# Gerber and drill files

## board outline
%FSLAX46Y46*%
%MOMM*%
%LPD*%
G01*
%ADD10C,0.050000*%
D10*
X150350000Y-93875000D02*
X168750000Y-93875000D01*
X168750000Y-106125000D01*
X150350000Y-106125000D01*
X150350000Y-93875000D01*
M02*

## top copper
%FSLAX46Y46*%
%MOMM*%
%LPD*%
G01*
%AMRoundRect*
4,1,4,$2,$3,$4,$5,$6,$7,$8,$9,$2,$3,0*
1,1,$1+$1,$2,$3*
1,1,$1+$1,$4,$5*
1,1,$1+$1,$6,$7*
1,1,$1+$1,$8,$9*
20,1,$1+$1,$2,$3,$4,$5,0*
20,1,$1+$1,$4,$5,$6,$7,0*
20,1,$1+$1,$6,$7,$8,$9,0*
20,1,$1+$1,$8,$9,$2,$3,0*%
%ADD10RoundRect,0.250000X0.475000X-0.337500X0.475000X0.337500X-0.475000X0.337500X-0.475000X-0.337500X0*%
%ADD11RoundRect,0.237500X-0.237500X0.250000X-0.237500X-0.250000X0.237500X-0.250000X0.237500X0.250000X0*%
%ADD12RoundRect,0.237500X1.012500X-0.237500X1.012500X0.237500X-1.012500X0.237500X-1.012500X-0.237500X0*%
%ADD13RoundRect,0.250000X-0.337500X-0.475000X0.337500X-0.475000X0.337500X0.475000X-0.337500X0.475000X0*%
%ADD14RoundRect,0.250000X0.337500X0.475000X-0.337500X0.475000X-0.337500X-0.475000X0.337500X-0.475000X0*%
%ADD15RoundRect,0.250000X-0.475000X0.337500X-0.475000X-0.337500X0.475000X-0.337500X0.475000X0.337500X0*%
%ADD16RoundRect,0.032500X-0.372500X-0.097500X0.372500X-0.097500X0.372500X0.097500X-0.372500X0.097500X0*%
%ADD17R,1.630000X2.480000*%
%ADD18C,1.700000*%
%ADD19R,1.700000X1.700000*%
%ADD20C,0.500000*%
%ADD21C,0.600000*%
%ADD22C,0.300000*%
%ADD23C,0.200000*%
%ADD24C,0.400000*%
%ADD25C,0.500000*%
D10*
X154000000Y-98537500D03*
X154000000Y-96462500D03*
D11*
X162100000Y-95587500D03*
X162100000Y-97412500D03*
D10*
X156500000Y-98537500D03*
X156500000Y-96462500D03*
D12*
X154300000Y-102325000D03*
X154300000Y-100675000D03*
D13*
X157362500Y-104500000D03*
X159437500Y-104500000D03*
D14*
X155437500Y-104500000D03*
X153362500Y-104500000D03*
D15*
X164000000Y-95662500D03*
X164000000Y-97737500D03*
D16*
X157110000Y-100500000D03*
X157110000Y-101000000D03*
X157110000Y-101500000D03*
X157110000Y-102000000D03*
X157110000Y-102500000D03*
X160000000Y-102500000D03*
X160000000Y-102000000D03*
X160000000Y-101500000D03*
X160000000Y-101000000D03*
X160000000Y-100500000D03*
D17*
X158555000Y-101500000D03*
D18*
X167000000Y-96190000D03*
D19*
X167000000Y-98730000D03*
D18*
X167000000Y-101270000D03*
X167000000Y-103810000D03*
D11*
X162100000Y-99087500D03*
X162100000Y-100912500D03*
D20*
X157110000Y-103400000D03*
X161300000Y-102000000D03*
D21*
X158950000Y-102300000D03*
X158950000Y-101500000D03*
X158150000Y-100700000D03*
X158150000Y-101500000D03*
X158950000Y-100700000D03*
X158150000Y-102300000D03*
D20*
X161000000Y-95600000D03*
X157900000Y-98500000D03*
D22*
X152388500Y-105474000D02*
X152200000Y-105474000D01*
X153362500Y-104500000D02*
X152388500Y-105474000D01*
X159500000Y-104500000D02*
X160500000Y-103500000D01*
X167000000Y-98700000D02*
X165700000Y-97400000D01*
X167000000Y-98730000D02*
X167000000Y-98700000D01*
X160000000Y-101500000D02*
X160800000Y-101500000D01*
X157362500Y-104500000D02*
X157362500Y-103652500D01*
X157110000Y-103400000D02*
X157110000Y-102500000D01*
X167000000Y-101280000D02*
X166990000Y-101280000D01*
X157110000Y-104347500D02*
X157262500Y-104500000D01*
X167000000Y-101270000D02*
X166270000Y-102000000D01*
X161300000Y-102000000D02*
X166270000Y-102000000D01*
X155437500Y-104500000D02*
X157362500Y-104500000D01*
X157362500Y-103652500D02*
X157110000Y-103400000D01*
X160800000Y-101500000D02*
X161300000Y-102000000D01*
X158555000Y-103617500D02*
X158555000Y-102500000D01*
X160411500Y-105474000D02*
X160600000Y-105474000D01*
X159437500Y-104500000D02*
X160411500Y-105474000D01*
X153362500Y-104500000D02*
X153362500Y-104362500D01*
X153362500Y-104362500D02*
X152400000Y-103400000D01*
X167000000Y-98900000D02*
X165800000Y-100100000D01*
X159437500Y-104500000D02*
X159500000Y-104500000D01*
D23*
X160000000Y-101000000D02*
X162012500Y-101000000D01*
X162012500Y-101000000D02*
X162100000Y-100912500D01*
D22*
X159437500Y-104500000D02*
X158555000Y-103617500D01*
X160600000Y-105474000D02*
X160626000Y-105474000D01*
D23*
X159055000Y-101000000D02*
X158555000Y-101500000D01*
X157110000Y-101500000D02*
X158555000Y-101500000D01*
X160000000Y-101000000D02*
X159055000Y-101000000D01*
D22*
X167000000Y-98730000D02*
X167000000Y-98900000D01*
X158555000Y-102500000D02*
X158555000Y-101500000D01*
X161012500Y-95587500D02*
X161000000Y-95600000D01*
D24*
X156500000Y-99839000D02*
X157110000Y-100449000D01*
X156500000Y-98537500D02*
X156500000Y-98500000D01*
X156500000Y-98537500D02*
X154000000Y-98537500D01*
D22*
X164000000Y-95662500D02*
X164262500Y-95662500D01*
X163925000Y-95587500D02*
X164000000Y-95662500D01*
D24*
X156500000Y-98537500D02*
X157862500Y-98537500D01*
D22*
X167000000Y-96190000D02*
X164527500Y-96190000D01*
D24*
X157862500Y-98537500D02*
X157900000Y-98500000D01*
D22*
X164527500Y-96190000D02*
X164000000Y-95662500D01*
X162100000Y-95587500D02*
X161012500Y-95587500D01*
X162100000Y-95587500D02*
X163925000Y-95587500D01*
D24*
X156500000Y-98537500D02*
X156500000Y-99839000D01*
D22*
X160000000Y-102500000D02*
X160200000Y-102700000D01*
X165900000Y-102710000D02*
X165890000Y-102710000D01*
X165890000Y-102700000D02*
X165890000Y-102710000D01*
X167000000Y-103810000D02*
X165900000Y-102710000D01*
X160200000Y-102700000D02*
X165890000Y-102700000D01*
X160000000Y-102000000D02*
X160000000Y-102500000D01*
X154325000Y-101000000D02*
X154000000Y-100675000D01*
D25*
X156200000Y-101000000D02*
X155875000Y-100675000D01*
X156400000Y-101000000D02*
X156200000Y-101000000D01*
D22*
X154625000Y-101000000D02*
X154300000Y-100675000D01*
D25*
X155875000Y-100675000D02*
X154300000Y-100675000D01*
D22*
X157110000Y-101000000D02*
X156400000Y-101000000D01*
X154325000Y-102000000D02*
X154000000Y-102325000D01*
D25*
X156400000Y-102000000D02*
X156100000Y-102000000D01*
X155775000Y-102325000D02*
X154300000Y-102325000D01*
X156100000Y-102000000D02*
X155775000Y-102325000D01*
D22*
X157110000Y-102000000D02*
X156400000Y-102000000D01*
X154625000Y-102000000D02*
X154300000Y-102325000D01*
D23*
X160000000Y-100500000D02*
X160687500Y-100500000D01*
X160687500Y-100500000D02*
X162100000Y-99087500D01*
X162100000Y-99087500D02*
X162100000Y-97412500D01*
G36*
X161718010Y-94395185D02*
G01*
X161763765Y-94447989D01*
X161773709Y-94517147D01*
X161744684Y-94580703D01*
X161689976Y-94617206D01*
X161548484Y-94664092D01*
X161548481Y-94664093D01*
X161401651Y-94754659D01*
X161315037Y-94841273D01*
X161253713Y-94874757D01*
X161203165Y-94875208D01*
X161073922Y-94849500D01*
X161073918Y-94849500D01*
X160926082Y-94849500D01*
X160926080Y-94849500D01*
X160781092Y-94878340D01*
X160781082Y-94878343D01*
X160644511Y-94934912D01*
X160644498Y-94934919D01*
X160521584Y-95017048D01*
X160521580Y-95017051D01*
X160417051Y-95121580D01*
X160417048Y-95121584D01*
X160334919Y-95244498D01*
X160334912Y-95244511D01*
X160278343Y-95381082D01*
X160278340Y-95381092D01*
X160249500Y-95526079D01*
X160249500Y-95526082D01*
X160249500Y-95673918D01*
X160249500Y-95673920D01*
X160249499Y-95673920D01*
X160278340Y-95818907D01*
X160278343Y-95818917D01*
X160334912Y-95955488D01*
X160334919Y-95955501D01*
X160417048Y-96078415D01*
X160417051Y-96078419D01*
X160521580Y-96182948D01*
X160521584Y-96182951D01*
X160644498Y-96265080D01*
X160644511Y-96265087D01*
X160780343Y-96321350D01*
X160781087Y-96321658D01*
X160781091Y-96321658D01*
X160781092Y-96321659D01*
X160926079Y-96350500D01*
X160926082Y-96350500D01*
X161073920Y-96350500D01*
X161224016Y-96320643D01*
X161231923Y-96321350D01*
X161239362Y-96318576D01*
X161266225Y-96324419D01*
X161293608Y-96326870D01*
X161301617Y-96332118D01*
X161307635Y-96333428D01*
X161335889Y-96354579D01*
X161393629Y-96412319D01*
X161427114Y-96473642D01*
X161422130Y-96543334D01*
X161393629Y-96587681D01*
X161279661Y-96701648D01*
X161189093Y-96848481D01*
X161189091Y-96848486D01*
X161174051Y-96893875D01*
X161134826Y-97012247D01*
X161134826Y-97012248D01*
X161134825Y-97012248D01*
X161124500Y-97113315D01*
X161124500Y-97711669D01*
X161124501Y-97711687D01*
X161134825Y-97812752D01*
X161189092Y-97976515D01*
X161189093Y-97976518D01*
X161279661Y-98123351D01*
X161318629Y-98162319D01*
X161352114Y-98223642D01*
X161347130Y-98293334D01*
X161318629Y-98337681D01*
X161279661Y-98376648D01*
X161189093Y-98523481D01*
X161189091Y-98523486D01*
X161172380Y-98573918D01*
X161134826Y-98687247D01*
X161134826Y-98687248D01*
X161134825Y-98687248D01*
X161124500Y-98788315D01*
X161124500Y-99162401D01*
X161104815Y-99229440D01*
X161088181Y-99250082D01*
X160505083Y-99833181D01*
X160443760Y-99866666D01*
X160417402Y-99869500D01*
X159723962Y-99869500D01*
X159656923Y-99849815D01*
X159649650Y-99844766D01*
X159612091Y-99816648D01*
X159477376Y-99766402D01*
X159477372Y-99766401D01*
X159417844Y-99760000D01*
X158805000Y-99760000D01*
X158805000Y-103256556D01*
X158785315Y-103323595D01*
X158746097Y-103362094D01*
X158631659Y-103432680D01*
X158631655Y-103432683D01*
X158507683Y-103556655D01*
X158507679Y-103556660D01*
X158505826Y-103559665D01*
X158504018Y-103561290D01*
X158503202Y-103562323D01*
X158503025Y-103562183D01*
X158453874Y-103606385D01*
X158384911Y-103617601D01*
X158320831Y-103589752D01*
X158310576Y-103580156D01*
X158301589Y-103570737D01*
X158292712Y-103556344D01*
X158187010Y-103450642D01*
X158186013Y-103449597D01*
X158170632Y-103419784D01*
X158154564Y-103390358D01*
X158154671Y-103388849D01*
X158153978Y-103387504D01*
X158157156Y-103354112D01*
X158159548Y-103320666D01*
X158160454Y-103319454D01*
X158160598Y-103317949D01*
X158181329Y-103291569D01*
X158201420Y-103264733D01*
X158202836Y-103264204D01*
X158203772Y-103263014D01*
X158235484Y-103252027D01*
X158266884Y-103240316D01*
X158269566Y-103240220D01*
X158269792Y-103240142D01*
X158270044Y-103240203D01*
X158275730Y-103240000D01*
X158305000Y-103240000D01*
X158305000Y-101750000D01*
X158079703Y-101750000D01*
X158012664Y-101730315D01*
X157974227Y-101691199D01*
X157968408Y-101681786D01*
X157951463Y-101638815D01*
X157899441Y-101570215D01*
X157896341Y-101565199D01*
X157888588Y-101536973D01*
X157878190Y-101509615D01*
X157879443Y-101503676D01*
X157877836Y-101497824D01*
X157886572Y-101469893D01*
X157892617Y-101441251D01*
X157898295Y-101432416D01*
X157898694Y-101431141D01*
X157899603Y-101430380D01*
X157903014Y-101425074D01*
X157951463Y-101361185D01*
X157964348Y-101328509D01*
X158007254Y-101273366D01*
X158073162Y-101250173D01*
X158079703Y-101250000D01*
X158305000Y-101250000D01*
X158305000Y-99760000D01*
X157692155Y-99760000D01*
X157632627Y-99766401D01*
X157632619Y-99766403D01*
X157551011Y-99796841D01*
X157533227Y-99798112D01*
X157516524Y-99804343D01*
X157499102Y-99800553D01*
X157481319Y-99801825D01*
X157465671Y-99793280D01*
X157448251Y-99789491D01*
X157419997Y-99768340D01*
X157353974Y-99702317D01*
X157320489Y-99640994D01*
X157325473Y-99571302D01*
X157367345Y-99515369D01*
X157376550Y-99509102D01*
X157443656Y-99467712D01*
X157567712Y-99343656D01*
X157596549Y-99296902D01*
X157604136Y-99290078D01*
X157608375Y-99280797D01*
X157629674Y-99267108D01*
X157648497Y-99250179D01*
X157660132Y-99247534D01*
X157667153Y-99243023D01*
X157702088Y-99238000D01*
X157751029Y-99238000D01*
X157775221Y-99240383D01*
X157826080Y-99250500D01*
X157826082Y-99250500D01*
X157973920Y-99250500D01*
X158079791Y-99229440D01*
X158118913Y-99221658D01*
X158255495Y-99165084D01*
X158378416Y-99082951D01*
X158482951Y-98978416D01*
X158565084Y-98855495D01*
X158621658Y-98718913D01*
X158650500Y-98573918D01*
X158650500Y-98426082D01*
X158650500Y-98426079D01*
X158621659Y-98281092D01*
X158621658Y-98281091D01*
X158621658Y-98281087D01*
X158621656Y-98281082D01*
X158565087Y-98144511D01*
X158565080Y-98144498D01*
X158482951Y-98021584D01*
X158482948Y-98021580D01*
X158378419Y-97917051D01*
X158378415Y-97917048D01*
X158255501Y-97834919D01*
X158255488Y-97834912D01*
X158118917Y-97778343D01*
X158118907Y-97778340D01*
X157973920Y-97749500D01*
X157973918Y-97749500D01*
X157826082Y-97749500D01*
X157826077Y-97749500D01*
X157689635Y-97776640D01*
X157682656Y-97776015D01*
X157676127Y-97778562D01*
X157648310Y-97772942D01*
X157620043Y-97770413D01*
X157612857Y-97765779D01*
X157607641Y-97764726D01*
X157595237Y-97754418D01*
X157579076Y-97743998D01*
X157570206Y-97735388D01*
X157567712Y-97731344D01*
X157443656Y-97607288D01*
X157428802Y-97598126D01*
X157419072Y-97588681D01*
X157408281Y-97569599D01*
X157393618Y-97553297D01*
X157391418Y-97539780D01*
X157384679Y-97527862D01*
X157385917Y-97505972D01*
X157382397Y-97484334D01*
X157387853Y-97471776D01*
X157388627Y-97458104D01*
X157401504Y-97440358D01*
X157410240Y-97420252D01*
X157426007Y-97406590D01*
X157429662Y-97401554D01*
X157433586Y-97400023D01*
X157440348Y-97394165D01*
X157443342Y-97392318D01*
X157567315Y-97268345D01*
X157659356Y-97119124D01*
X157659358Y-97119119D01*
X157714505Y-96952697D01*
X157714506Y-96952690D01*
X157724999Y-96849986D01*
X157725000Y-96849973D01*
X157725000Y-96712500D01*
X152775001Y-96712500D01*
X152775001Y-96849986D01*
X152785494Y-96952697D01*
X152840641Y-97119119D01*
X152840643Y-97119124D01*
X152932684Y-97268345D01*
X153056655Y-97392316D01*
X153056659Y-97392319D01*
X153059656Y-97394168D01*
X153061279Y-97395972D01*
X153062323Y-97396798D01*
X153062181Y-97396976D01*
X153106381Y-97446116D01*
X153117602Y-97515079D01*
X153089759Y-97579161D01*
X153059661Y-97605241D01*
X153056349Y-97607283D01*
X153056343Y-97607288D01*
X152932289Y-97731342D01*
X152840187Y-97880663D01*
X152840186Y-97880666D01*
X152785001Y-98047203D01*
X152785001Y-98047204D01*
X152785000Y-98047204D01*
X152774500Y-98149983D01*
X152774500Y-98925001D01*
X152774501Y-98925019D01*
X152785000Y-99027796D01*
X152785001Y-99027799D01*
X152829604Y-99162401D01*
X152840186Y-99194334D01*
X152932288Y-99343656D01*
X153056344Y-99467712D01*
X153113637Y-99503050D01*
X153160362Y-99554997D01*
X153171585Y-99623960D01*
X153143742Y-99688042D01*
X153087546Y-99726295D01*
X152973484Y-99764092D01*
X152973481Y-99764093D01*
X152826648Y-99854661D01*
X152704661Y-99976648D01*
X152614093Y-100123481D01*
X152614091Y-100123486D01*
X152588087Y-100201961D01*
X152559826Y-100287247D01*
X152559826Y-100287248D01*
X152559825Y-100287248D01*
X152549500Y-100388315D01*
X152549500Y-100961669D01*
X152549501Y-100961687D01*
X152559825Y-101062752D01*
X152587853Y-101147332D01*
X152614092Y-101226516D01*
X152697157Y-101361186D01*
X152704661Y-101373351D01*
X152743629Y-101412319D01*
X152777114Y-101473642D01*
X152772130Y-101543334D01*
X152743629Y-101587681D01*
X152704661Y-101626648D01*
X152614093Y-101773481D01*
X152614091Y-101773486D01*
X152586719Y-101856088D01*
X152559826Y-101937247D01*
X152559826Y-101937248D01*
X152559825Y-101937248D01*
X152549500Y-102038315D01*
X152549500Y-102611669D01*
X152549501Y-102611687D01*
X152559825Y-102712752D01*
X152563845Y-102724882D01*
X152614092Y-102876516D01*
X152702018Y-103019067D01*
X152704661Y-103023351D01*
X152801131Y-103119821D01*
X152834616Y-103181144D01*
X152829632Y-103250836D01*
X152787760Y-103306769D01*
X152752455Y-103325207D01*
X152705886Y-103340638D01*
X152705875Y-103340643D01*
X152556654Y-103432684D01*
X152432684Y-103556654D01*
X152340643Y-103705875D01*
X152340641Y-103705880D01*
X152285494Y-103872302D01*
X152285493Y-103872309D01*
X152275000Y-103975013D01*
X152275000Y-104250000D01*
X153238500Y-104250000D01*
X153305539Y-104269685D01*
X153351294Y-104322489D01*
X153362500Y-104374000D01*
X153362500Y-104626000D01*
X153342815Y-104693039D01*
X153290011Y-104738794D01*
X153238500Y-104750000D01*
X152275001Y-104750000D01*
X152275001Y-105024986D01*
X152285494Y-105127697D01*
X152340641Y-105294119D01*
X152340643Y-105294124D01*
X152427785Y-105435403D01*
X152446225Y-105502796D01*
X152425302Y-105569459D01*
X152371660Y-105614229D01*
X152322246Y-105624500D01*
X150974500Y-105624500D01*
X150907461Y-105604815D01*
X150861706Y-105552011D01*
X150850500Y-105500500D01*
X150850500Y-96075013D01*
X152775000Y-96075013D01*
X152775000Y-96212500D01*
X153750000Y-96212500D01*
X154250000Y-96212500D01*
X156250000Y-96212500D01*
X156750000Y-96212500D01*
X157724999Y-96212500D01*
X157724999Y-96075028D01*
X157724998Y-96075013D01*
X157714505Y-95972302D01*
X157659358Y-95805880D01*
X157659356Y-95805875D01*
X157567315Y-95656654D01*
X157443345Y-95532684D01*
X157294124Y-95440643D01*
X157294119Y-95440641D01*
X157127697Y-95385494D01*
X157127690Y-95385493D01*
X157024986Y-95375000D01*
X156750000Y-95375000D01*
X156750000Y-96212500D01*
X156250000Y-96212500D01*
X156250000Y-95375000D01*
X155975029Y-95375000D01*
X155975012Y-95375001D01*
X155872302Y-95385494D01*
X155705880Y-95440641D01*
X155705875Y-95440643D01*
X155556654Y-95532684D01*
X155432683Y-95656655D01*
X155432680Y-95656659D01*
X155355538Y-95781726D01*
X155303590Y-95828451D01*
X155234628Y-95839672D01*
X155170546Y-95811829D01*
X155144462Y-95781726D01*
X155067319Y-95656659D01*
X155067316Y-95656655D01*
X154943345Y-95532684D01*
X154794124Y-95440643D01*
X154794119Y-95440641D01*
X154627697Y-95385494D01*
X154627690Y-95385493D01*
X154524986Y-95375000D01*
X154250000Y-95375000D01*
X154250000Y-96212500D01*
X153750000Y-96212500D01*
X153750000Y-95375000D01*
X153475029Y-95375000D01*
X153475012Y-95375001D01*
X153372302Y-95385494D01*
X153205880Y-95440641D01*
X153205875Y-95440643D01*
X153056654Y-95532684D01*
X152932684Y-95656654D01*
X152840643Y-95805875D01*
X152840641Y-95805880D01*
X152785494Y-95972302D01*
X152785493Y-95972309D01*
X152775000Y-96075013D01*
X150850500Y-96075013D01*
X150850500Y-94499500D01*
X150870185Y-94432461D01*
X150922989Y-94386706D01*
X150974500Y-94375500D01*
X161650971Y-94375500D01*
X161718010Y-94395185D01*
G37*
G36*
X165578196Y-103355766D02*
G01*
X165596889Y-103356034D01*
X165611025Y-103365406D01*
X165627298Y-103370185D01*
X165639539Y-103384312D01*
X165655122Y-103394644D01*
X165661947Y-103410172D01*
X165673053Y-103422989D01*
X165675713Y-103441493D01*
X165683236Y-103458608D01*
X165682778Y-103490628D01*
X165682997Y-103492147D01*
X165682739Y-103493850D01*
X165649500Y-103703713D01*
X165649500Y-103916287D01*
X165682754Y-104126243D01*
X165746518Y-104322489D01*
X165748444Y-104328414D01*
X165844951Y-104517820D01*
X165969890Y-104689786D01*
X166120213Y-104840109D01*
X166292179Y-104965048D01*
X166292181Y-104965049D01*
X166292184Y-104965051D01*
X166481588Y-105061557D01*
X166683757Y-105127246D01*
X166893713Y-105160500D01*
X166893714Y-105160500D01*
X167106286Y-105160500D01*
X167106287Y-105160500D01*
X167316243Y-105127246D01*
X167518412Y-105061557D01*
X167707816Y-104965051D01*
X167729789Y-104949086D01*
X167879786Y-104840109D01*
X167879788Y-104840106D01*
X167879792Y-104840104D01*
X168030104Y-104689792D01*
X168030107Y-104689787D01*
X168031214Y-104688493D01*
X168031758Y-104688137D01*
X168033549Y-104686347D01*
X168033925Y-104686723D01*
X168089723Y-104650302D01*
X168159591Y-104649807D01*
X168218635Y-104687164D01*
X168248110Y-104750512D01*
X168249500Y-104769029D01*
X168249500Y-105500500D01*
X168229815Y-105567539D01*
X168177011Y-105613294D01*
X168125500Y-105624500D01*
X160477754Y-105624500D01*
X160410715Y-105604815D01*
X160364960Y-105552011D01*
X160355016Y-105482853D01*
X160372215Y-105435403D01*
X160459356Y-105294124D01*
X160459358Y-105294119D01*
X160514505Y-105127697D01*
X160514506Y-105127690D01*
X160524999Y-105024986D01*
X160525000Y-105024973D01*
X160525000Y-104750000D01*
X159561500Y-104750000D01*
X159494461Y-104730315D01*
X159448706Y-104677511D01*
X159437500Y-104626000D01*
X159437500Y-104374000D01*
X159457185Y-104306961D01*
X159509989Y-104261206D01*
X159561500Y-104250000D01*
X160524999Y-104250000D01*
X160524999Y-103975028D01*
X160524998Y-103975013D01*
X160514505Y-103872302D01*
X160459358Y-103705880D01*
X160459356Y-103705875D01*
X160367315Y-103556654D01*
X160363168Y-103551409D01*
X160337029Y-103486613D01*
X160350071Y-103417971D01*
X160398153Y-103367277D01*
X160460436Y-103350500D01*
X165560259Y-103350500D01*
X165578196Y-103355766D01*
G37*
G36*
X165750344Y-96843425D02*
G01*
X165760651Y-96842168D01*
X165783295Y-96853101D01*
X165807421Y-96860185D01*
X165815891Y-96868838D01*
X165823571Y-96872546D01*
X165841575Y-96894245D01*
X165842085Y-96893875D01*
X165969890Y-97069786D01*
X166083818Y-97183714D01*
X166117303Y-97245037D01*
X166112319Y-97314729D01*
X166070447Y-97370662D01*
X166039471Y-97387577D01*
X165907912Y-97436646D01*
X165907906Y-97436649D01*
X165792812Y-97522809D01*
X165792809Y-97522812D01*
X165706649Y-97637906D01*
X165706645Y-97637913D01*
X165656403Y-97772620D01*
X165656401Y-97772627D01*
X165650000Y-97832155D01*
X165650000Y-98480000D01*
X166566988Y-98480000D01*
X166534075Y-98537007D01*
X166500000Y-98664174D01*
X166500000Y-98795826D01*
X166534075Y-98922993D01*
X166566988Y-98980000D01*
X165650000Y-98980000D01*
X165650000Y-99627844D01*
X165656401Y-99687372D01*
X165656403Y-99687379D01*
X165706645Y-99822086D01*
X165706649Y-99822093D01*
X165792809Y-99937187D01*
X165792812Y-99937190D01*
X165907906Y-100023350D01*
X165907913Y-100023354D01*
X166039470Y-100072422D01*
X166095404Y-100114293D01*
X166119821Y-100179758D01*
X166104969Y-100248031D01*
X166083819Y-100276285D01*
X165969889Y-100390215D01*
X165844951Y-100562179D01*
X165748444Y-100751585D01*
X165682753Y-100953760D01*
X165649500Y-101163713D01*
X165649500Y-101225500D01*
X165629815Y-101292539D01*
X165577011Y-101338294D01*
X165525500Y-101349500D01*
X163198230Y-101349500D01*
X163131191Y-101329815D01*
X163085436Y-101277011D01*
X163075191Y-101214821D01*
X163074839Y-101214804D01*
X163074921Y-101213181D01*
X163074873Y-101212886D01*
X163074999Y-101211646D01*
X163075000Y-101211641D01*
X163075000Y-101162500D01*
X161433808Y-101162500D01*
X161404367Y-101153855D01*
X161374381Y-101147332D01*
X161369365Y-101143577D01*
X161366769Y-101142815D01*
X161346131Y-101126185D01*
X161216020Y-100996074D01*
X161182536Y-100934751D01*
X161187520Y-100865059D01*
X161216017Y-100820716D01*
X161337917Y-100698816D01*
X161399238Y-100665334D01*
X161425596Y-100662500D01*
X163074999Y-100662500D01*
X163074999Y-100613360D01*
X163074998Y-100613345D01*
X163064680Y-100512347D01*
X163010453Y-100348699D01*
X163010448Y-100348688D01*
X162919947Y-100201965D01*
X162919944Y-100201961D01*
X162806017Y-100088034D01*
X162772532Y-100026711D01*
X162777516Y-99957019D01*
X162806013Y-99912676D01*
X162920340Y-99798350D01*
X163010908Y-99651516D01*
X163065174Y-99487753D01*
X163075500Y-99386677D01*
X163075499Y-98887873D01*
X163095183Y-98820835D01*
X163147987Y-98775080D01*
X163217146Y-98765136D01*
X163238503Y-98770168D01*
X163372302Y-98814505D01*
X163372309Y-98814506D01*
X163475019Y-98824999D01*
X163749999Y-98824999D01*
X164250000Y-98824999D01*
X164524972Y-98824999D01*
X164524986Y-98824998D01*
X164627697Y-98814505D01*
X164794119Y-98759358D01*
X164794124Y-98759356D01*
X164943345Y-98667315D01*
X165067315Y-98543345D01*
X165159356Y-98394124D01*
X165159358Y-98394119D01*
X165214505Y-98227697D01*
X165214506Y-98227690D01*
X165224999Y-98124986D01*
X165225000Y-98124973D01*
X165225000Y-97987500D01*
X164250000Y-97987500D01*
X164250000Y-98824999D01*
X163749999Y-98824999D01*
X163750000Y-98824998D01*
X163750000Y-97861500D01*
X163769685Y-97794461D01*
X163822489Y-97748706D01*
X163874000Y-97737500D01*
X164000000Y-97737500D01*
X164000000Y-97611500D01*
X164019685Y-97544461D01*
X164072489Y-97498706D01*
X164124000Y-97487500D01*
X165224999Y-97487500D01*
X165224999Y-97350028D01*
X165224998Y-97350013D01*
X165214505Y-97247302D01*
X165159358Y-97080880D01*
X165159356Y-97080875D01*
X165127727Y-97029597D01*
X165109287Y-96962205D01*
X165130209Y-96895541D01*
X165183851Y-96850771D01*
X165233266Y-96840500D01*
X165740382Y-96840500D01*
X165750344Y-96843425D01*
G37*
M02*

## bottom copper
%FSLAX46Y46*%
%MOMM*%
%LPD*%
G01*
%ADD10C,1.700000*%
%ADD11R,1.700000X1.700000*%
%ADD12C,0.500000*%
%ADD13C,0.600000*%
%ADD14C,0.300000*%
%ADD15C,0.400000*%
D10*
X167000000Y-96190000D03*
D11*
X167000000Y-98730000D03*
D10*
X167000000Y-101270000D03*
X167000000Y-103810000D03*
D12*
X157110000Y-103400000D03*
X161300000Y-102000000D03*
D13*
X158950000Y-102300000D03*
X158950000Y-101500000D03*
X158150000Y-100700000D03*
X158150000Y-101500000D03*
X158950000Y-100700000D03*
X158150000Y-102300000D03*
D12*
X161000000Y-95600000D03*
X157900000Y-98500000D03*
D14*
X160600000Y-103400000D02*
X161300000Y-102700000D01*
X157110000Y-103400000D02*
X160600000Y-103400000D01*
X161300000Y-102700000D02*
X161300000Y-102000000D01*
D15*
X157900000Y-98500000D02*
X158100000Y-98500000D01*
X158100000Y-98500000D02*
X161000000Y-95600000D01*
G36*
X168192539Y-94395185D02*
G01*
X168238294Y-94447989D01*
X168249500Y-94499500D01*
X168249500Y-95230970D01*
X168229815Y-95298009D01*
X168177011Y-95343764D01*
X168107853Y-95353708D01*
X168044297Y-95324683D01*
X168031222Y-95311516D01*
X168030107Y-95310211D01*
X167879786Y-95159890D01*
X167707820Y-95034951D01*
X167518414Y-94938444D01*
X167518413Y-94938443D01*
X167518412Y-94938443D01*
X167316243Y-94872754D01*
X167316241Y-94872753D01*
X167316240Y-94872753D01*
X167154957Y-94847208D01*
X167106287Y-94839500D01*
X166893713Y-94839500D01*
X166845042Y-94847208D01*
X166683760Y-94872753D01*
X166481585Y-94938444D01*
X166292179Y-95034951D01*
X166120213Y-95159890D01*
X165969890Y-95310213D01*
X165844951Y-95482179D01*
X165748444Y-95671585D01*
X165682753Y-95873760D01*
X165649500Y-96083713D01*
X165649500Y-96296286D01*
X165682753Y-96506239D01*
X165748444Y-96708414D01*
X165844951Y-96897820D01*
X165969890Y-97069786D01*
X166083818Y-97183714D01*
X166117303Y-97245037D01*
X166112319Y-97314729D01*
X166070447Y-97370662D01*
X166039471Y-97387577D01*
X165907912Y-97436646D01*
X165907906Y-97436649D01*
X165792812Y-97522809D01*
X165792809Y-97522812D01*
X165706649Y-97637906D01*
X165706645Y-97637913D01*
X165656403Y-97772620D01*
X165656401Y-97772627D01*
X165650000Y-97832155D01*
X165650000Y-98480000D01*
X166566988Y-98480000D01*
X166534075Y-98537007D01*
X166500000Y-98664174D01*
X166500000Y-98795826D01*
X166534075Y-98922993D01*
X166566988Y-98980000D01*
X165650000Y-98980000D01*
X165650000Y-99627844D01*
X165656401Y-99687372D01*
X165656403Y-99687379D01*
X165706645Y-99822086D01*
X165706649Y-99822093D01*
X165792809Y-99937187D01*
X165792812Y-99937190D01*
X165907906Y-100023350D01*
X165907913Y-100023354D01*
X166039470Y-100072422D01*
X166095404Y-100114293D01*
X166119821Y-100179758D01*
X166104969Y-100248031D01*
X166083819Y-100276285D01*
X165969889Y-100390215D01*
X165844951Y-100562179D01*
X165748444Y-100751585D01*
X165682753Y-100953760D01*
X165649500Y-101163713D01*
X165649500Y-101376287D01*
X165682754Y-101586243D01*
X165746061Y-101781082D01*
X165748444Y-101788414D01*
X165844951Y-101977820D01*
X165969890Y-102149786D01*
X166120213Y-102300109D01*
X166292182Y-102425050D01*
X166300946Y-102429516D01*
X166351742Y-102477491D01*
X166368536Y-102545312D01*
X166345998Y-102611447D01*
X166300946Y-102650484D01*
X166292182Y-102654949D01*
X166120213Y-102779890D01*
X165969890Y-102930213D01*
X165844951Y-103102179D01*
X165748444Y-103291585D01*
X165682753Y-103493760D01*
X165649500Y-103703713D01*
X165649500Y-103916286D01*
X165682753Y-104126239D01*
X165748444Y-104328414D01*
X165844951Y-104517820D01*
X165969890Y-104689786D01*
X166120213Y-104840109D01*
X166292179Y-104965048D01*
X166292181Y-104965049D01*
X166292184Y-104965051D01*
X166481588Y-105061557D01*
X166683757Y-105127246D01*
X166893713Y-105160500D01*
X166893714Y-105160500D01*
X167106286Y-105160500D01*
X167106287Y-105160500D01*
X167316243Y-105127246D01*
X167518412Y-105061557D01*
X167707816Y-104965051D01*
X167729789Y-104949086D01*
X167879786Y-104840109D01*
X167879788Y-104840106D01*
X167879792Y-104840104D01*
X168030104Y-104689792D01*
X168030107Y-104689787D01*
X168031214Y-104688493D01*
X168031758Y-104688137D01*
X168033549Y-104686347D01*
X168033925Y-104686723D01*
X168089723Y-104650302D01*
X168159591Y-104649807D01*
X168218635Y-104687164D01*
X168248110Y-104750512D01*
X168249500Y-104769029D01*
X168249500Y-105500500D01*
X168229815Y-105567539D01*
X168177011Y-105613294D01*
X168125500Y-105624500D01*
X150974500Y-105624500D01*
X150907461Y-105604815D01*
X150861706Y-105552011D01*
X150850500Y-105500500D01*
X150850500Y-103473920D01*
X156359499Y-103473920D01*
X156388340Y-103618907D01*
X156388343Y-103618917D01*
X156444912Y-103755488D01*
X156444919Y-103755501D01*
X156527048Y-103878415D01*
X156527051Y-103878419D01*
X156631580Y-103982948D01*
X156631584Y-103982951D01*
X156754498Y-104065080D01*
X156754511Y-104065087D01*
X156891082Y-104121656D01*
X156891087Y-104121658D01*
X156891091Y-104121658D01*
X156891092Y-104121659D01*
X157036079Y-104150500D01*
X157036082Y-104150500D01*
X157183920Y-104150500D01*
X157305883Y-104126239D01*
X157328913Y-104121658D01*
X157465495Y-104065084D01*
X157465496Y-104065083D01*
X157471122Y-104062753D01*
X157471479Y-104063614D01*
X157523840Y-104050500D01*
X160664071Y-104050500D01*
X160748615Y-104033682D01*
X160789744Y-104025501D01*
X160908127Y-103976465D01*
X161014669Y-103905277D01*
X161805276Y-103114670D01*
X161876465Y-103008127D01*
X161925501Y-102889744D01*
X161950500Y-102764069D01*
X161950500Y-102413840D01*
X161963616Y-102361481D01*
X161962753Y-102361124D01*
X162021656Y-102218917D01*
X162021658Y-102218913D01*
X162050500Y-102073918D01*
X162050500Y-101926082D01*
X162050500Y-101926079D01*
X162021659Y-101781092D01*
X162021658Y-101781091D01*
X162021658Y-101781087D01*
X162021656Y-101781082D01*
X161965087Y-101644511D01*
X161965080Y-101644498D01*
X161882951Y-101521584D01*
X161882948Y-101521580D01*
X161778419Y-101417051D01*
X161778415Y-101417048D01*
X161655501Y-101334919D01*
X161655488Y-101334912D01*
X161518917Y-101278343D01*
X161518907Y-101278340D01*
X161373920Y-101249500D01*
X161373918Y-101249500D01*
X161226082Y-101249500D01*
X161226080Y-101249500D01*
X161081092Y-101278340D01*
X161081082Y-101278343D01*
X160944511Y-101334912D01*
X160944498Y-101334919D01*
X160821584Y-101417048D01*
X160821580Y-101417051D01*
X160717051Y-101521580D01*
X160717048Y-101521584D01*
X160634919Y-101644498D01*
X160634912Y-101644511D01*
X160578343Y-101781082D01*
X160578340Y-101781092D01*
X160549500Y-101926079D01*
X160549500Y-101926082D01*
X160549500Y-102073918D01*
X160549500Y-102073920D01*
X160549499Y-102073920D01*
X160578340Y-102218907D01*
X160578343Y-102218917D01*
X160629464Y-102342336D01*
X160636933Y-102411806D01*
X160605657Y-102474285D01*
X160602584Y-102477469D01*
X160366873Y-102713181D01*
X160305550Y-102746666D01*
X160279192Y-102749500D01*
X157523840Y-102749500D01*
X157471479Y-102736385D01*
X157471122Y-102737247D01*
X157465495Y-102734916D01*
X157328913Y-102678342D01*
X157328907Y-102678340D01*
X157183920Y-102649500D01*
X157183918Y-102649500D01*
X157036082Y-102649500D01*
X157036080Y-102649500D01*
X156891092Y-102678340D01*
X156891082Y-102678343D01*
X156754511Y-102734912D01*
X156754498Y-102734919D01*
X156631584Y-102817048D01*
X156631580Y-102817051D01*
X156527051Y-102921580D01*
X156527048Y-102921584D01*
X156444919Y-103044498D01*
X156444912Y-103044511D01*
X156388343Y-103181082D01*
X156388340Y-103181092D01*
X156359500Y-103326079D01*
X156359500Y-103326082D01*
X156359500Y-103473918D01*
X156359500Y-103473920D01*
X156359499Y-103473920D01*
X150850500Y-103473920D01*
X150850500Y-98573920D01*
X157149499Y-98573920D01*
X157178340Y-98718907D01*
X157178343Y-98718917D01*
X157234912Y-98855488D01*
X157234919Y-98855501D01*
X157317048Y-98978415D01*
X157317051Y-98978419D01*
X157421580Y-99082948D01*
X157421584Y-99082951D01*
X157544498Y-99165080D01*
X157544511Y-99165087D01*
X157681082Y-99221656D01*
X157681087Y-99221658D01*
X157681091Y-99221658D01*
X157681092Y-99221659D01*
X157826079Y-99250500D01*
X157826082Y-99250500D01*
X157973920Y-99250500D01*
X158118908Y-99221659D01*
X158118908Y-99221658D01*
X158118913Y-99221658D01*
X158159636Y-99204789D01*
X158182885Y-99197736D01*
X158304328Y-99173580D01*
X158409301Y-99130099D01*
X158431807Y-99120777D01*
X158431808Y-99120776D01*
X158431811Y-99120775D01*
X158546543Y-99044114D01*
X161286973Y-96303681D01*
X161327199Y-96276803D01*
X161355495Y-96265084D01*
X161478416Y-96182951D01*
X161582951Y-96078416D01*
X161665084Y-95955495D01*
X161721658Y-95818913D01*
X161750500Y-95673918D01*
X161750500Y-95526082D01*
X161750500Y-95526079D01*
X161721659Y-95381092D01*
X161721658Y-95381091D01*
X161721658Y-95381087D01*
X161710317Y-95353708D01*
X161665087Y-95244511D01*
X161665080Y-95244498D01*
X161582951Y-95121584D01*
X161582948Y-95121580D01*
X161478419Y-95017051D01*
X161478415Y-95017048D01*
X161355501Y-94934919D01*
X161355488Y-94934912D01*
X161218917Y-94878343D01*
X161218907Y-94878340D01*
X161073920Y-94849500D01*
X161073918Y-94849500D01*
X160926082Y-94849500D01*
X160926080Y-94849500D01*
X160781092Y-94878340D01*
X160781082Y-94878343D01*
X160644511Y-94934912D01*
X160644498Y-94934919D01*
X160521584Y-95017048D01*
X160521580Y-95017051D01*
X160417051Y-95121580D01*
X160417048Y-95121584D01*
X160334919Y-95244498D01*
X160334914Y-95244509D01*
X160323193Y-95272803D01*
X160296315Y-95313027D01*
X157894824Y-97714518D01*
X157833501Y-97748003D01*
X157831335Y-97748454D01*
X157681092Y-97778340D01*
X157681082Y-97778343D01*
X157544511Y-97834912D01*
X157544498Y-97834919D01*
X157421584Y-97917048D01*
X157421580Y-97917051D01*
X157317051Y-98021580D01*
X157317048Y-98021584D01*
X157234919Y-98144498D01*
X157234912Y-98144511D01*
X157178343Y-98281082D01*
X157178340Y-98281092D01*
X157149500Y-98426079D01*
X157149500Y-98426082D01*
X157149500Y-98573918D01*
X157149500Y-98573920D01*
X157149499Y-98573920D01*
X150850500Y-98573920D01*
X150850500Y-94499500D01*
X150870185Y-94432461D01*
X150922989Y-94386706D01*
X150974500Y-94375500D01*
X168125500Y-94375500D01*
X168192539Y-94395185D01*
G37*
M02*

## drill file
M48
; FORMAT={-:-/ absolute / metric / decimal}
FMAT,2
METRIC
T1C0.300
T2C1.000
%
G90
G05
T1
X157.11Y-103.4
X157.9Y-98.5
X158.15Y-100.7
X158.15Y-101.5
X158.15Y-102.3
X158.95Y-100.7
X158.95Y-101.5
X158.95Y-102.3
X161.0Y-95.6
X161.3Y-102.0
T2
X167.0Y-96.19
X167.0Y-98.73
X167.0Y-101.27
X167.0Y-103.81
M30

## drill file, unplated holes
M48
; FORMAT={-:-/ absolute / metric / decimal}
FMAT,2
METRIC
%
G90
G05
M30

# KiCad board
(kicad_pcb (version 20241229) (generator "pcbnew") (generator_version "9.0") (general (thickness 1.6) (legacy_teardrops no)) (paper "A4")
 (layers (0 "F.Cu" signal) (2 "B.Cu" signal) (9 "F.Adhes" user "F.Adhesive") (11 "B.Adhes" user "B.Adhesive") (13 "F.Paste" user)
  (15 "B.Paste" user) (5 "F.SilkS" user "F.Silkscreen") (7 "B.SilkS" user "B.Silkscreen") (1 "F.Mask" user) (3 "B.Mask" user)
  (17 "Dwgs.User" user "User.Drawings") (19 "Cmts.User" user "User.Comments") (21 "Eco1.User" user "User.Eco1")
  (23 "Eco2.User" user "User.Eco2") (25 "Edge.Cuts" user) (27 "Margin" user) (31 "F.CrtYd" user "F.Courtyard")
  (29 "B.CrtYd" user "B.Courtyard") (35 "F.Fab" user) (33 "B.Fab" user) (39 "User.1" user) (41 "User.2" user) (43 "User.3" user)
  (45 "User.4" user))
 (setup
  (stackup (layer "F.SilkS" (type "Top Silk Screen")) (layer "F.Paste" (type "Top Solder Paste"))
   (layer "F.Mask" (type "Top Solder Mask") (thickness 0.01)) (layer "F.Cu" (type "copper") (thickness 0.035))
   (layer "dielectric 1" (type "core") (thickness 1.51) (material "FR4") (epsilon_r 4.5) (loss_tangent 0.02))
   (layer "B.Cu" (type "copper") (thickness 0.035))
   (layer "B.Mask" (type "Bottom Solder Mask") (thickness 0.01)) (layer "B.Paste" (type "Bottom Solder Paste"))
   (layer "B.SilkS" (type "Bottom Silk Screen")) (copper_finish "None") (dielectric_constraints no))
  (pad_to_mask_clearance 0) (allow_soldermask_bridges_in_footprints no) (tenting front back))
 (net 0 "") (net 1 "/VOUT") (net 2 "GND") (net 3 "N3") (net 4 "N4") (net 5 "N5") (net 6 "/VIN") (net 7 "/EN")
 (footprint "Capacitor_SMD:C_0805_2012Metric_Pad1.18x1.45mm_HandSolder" (layer "F.Cu") (at 154 97.5 90)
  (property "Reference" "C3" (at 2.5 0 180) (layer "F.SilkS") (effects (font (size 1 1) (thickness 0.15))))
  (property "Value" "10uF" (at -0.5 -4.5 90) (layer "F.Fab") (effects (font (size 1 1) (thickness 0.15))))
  (pad "1" smd roundrect (at -1.0375 0 90) (size 1.175 1.45) (layers "F.Cu" "F.Mask" "F.Paste") (roundrect_rratio 0.212766) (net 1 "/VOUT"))
  (pad "2" smd roundrect (at 1.0375 0 90) (size 1.175 1.45) (layers "F.Cu" "F.Mask" "F.Paste") (roundrect_rratio 0.212766) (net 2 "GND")))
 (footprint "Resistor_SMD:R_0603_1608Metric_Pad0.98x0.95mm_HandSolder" (layer "F.Cu") (at 162.1 96.5 -90)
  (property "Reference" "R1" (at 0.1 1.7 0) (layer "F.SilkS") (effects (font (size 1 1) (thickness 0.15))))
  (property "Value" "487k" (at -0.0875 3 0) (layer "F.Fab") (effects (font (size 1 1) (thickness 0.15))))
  (pad "1" smd roundrect (at -0.9125 0 270) (size 0.975 0.95) (layers "F.Cu" "F.Mask" "F.Paste") (roundrect_rratio 0.25) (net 1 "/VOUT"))
  (pad "2" smd roundrect (at 0.9125 0 270) (size 0.975 0.95) (layers "F.Cu" "F.Mask" "F.Paste") (roundrect_rratio 0.25) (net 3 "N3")))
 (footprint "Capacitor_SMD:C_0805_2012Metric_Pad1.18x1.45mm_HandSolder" (layer "F.Cu") (at 156.5 97.5 90)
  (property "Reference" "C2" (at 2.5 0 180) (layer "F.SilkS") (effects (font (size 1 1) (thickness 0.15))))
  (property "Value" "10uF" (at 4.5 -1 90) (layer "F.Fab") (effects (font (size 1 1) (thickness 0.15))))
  (pad "1" smd roundrect (at -1.0375 0 90) (size 1.175 1.45) (layers "F.Cu" "F.Mask" "F.Paste") (roundrect_rratio 0.212766) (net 1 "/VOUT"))
  (pad "2" smd roundrect (at 1.0375 0 90) (size 1.175 1.45) (layers "F.Cu" "F.Mask" "F.Paste") (roundrect_rratio 0.212766) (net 2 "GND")))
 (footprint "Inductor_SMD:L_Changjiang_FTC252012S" (layer "F.Cu") (at 154.3 101.5 90)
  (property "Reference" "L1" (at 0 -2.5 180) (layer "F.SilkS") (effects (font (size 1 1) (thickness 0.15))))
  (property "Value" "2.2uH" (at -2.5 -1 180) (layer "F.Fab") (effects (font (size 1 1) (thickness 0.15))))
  (pad "1" smd roundrect (at -0.825 0 90) (size 0.95 2.5) (layers "F.Cu" "F.Mask" "F.Paste") (roundrect_rratio 0.25) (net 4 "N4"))
  (pad "2" smd roundrect (at 0.825 0 90) (size 0.95 2.5) (layers "F.Cu" "F.Mask" "F.Paste") (roundrect_rratio 0.25) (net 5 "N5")))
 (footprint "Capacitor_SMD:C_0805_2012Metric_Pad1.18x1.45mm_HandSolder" (layer "F.Cu") (at 158.4 104.5)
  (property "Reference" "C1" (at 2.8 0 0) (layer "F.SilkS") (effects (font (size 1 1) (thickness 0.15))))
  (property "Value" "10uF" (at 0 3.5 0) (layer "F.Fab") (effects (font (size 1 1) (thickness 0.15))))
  (pad "1" smd roundrect (at -1.0375 0) (size 1.175 1.45) (layers "F.Cu" "F.Mask" "F.Paste") (roundrect_rratio 0.212766) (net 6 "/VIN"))
  (pad "2" smd roundrect (at 1.0375 0) (size 1.175 1.45) (layers "F.Cu" "F.Mask" "F.Paste") (roundrect_rratio 0.212766) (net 2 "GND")))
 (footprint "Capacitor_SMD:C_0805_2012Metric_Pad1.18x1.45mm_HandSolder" (layer "F.Cu") (at 154.4 104.5 180)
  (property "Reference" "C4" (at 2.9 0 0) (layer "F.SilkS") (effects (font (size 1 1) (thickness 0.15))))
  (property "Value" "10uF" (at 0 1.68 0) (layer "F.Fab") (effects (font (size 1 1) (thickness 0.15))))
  (pad "1" smd roundrect (at -1.0375 0 180) (size 1.175 1.45) (layers "F.Cu" "F.Mask" "F.Paste") (roundrect_rratio 0.212766) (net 6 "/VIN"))
  (pad "2" smd roundrect (at 1.0375 0 180) (size 1.175 1.45) (layers "F.Cu" "F.Mask" "F.Paste") (roundrect_rratio 0.212766) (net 2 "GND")))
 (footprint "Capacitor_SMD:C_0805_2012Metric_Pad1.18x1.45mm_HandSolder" (layer "F.Cu") (at 164 96.7 -90)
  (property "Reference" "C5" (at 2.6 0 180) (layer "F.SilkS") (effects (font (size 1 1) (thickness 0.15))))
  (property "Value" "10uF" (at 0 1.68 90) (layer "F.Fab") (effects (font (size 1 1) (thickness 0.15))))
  (pad "1" smd roundrect (at -1.0375 0 270) (size 1.175 1.45) (layers "F.Cu" "F.Mask" "F.Paste") (roundrect_rratio 0.212766) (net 1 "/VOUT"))
  (pad "2" smd roundrect (at 1.0375 0 270) (size 1.175 1.45) (layers "F.Cu" "F.Mask" "F.Paste") (roundrect_rratio 0.212766) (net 2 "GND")))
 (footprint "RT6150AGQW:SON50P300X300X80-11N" (layer "F.Cu") (at 158.555 101.5)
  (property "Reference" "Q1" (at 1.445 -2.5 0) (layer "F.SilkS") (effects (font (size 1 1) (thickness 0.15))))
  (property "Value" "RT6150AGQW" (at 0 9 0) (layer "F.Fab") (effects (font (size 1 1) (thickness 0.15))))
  (pad "1" smd roundrect (at -1.445 -1) (size 0.81 0.26) (layers "F.Cu" "F.Mask" "F.Paste") (roundrect_rratio 0.125) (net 1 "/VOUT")
   (solder_mask_margin 0.102))
  (pad "2" smd roundrect (at -1.445 -0.5) (size 0.81 0.26) (layers "F.Cu" "F.Mask" "F.Paste") (roundrect_rratio 0.125) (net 5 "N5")
   (solder_mask_margin 0.102))
  (pad "3" smd roundrect (at -1.445 0) (size 0.81 0.26) (layers "F.Cu" "F.Mask" "F.Paste") (roundrect_rratio 0.125) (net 2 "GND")
   (solder_mask_margin 0.102))
  (pad "4" smd roundrect (at -1.445 0.5) (size 0.81 0.26) (layers "F.Cu" "F.Mask" "F.Paste") (roundrect_rratio 0.125) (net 4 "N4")
   (solder_mask_margin 0.102))
  (pad "5" smd roundrect (at -1.445 1) (size 0.81 0.26) (layers "F.Cu" "F.Mask" "F.Paste") (roundrect_rratio 0.125) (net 6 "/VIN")
   (solder_mask_margin 0.102))
  (pad "6" smd roundrect (at 1.445 1) (size 0.81 0.26) (layers "F.Cu" "F.Mask" "F.Paste") (roundrect_rratio 0.125) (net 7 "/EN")
   (solder_mask_margin 0.102))
  (pad "7" smd roundrect (at 1.445 0.5) (size 0.81 0.26) (layers "F.Cu" "F.Mask" "F.Paste") (roundrect_rratio 0.125) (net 7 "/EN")
   (solder_mask_margin 0.102))
  (pad "8" smd roundrect (at 1.445 0) (size 0.81 0.26) (layers "F.Cu" "F.Mask" "F.Paste") (roundrect_rratio 0.125) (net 6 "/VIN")
   (solder_mask_margin 0.102))
  (pad "9" smd roundrect (at 1.445 -0.5) (size 0.81 0.26) (layers "F.Cu" "F.Mask" "F.Paste") (roundrect_rratio 0.125) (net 2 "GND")
   (solder_mask_margin 0.102))
  (pad "10" smd roundrect (at 1.445 -1) (size 0.81 0.26) (layers "F.Cu" "F.Mask" "F.Paste") (roundrect_rratio 0.125) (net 3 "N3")
   (solder_mask_margin 0.102))
  (pad "11" smd rect (at 0 0) (size 1.63 2.48) (layers "F.Cu" "F.Mask") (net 2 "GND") (solder_mask_margin 0.102)))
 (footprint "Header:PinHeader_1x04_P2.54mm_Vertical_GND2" (layer "F.Cu") (at 167 96.19)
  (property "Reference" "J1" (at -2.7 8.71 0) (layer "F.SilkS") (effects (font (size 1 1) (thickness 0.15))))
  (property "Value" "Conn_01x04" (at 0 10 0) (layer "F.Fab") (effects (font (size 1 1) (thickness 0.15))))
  (pad "1" thru_hole circle (at 0 0) (size 1.7 1.7) (drill 1) (layers "*.Cu" "*.Mask") (remove_unused_layers no) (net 1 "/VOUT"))
  (pad "2" thru_hole rect (at 0 2.54) (size 1.7 1.7) (drill 1) (layers "*.Cu" "*.Mask") (remove_unused_layers no) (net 2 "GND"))
  (pad "3" thru_hole circle (at 0 5.08) (size 1.7 1.7) (drill 1) (layers "*.Cu" "*.Mask") (remove_unused_layers no) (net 6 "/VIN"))
  (pad "4" thru_hole circle (at 0 7.62) (size 1.7 1.7) (drill 1) (layers "*.Cu" "*.Mask") (remove_unused_layers no) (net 7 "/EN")))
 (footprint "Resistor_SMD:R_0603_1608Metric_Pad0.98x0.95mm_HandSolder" (layer "F.Cu") (at 162.1 100 -90)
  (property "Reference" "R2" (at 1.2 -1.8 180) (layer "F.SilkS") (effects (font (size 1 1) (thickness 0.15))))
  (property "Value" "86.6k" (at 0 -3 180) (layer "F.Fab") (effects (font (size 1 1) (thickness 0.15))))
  (pad "1" smd roundrect (at -0.9125 0 270) (size 0.975 0.95) (layers "F.Cu" "F.Mask" "F.Paste") (roundrect_rratio 0.25) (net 3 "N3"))
  (pad "2" smd roundrect (at 0.9125 0 270) (size 0.975 0.95) (layers "F.Cu" "F.Mask" "F.Paste") (roundrect_rratio 0.25) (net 2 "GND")))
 (gr_rect (start 150.35 93.875) (end 168.75 106.125) (stroke (width 0.05) (type default)) (fill no) (layer "Edge.Cuts"))
 (segment (start 160 101.5) (end 160.8 101.5) (width 0.3) (layer "F.Cu") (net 6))
 (segment (start 157.3625 104.5) (end 157.3625 103.6525) (width 0.3) (layer "F.Cu") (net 6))
 (segment (start 157.11 103.4) (end 157.11 102.5) (width 0.3) (layer "F.Cu") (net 6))
 (segment (start 167 101.28) (end 166.99 101.28) (width 0.3) (layer "F.Cu") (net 6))
 (segment (start 157.11 104.3475) (end 157.2625 104.5) (width 0.3) (layer "F.Cu") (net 6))
 (segment (start 167 101.27) (end 166.27 102) (width 0.3) (layer "F.Cu") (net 6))
 (segment (start 161.3 102) (end 166.27 102) (width 0.3) (layer "F.Cu") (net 6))
 (segment (start 155.4375 104.5) (end 157.3625 104.5) (width 0.3) (layer "F.Cu") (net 6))
 (segment (start 157.3625 103.6525) (end 157.11 103.4) (width 0.3) (layer "F.Cu") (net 6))
 (segment (start 160.8 101.5) (end 161.3 102) (width 0.3) (layer "F.Cu") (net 6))
 (via (at 157.11 103.4) (size 0.5) (drill 0.3) (layers "F.Cu" "B.Cu") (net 6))
 (via (at 161.3 102) (size 0.5) (drill 0.3) (layers "F.Cu" "B.Cu") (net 6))
 (segment (start 160.6 103.4) (end 161.3 102.7) (width 0.3) (layer "B.Cu") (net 6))
 (segment (start 157.11 103.4) (end 160.6 103.4) (width 0.3) (layer "B.Cu") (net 6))
 (segment (start 161.3 102.7) (end 161.3 102) (width 0.3) (layer "B.Cu") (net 6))
 (segment (start 158.555 103.6175) (end 158.555 102.5) (width 0.3) (layer "F.Cu") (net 2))
 (segment (start 160.4115 105.474) (end 160.6 105.474) (width 0.3) (layer "F.Cu") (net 2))
 (segment (start 159.4375 104.5) (end 160.4115 105.474) (width 0.3) (layer "F.Cu") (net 2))
 (segment (start 153.3625 104.5) (end 153.3625 104.3625) (width 0.3) (layer "F.Cu") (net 2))
 (segment (start 153.3625 104.3625) (end 152.4 103.4) (width 0.3) (layer "F.Cu") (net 2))
 (segment (start 152.3885 105.474) (end 152.2 105.474) (width 0.3) (layer "F.Cu") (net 2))
 (segment (start 167 98.7) (end 165.7 97.4) (width 0.3) (layer "F.Cu") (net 2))
 (segment (start 167 98.9) (end 165.8 100.1) (width 0.3) (layer "F.Cu") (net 2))
 (segment (start 159.4375 104.5) (end 159.5 104.5) (width 0.3) (layer "F.Cu") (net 2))
 (segment (start 160 101) (end 162.0125 101) (width 0.2) (layer "F.Cu") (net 2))
 (segment (start 162.0125 101) (end 162.1 100.9125) (width 0.2) (layer "F.Cu") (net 2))
 (segment (start 153.3625 104.5) (end 152.3885 105.474) (width 0.3) (layer "F.Cu") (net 2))
 (segment (start 159.4375 104.5) (end 158.555 103.6175) (width 0.3) (layer "F.Cu") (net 2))
 (segment (start 160.6 105.474) (end 160.626 105.474) (width 0.3) (layer "F.Cu") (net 2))
 (segment (start 159.055 101) (end 158.555 101.5) (width 0.2) (layer "F.Cu") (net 2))
 (segment (start 159.5 104.5) (end 160.5 103.5) (width 0.3) (layer "F.Cu") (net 2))
 (segment (start 167 98.73) (end 167 98.7) (width 0.3) (layer "F.Cu") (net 2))
 (segment (start 157.11 101.5) (end 158.555 101.5) (width 0.2) (layer "F.Cu") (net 2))
 (segment (start 160 101) (end 159.055 101) (width 0.2) (layer "F.Cu") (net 2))
 (segment (start 167 98.73) (end 167 98.9) (width 0.3) (layer "F.Cu") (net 2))
 (segment (start 158.555 102.5) (end 158.555 101.5) (width 0.3) (layer "F.Cu") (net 2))
 (via (at 158.95 102.3) (size 0.6) (drill 0.3) (layers "F.Cu" "B.Cu") (tenting none) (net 2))
 (via (at 158.95 101.5) (size 0.6) (drill 0.3) (layers "F.Cu" "B.Cu") (tenting none) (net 2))
 (via (at 158.15 100.7) (size 0.6) (drill 0.3) (layers "F.Cu" "B.Cu") (tenting none) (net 2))
 (via (at 158.15 101.5) (size 0.6) (drill 0.3) (layers "F.Cu" "B.Cu") (tenting none) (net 2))
 (via (at 158.95 100.7) (size 0.6) (drill 0.3) (layers "F.Cu" "B.Cu") (tenting none) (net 2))
 (via (at 158.15 102.3) (size 0.6) (drill 0.3) (layers "F.Cu" "B.Cu") (tenting none) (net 2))
 (segment (start 161.0125 95.5875) (end 161 95.6) (width 0.3) (layer "F.Cu") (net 1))
 (segment (start 156.5 99.839) (end 157.11 100.449) (width 0.4) (layer "F.Cu") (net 1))
 (segment (start 156.5 98.5375) (end 156.5 98.5) (width 0.4) (layer "F.Cu") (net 1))
 (segment (start 156.5 98.5375) (end 154 98.5375) (width 0.4) (layer "F.Cu") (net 1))
 (segment (start 164 95.6625) (end 164.2625 95.6625) (width 0.3) (layer "F.Cu") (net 1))
 (segment (start 163.925 95.5875) (end 164 95.6625) (width 0.3) (layer "F.Cu") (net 1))
 (segment (start 156.5 98.5375) (end 157.8625 98.5375) (width 0.4) (layer "F.Cu") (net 1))
 (segment (start 167 96.19) (end 164.5275 96.19) (width 0.3) (layer "F.Cu") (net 1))
 (segment (start 157.8625 98.5375) (end 157.9 98.5) (width 0.4) (layer "F.Cu") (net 1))
 (segment (start 164.5275 96.19) (end 164 95.6625) (width 0.3) (layer "F.Cu") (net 1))
 (segment (start 162.1 95.5875) (end 161.0125 95.5875) (width 0.3) (layer "F.Cu") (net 1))
 (segment (start 162.1 95.5875) (end 163.925 95.5875) (width 0.3) (layer "F.Cu") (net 1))
 (segment (start 156.5 98.5375) (end 156.5 99.839) (width 0.4) (layer "F.Cu") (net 1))
 (via (at 161 95.6) (size 0.5) (drill 0.3) (layers "F.Cu" "B.Cu") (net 1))
 (via (at 157.9 98.5) (size 0.5) (drill 0.3) (layers "F.Cu" "B.Cu") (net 1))
 (segment (start 157.9 98.5) (end 158.1 98.5) (width 0.4) (layer "B.Cu") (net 1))
 (segment (start 158.1 98.5) (end 161 95.6) (width 0.4) (layer "B.Cu") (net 1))
 (segment (start 160 102.5) (end 160.2 102.7) (width 0.3) (layer "F.Cu") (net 7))
 (segment (start 165.9 102.71) (end 165.89 102.71) (width 0.3) (layer "F.Cu") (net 7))
 (segment (start 165.89 102.7) (end 165.89 102.71) (width 0.3) (layer "F.Cu") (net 7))
 (segment (start 167 103.81) (end 165.9 102.71) (width 0.3) (layer "F.Cu") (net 7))
 (segment (start 160.2 102.7) (end 165.89 102.7) (width 0.3) (layer "F.Cu") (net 7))
 (segment (start 160 102) (end 160 102.5) (width 0.3) (layer "F.Cu") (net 7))
 (segment (start 154.325 101) (end 154 100.675) (width 0.3) (layer "F.Cu") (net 5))
 (segment (start 156.2 101) (end 155.875 100.675) (width 0.5) (layer "F.Cu") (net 5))
 (segment (start 156.4 101) (end 156.2 101) (width 0.5) (layer "F.Cu") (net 5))
 (segment (start 154.625 101) (end 154.3 100.675) (width 0.3) (layer "F.Cu") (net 5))
 (segment (start 155.875 100.675) (end 154.3 100.675) (width 0.5) (layer "F.Cu") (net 5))
 (segment (start 157.11 101) (end 156.4 101) (width 0.3) (layer "F.Cu") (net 5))
 (segment (start 154.325 102) (end 154 102.325) (width 0.3) (layer "F.Cu") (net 4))
 (segment (start 156.4 102) (end 156.1 102) (width 0.5) (layer "F.Cu") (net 4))
 (segment (start 155.775 102.325) (end 154.3 102.325) (width 0.5) (layer "F.Cu") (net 4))
 (segment (start 156.1 102) (end 155.775 102.325) (width 0.5) (layer "F.Cu") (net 4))
 (segment (start 157.11 102) (end 156.4 102) (width 0.3) (layer "F.Cu") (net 4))
 (segment (start 154.625 102) (end 154.3 102.325) (width 0.3) (layer "F.Cu") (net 4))
 (segment (start 160 100.5) (end 160.6875 100.5) (width 0.2) (layer "F.Cu") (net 3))
 (segment (start 160.6875 100.5) (end 162.1 99.0875) (width 0.2) (layer "F.Cu") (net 3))
 (segment (start 162.1 99.0875) (end 162.1 97.4125) (width 0.2) (layer "F.Cu") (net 3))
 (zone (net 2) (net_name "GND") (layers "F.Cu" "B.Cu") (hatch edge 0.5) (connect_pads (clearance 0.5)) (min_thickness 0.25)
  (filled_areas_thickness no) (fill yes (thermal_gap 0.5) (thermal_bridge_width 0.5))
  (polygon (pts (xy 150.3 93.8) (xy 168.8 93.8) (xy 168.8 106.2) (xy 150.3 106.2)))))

